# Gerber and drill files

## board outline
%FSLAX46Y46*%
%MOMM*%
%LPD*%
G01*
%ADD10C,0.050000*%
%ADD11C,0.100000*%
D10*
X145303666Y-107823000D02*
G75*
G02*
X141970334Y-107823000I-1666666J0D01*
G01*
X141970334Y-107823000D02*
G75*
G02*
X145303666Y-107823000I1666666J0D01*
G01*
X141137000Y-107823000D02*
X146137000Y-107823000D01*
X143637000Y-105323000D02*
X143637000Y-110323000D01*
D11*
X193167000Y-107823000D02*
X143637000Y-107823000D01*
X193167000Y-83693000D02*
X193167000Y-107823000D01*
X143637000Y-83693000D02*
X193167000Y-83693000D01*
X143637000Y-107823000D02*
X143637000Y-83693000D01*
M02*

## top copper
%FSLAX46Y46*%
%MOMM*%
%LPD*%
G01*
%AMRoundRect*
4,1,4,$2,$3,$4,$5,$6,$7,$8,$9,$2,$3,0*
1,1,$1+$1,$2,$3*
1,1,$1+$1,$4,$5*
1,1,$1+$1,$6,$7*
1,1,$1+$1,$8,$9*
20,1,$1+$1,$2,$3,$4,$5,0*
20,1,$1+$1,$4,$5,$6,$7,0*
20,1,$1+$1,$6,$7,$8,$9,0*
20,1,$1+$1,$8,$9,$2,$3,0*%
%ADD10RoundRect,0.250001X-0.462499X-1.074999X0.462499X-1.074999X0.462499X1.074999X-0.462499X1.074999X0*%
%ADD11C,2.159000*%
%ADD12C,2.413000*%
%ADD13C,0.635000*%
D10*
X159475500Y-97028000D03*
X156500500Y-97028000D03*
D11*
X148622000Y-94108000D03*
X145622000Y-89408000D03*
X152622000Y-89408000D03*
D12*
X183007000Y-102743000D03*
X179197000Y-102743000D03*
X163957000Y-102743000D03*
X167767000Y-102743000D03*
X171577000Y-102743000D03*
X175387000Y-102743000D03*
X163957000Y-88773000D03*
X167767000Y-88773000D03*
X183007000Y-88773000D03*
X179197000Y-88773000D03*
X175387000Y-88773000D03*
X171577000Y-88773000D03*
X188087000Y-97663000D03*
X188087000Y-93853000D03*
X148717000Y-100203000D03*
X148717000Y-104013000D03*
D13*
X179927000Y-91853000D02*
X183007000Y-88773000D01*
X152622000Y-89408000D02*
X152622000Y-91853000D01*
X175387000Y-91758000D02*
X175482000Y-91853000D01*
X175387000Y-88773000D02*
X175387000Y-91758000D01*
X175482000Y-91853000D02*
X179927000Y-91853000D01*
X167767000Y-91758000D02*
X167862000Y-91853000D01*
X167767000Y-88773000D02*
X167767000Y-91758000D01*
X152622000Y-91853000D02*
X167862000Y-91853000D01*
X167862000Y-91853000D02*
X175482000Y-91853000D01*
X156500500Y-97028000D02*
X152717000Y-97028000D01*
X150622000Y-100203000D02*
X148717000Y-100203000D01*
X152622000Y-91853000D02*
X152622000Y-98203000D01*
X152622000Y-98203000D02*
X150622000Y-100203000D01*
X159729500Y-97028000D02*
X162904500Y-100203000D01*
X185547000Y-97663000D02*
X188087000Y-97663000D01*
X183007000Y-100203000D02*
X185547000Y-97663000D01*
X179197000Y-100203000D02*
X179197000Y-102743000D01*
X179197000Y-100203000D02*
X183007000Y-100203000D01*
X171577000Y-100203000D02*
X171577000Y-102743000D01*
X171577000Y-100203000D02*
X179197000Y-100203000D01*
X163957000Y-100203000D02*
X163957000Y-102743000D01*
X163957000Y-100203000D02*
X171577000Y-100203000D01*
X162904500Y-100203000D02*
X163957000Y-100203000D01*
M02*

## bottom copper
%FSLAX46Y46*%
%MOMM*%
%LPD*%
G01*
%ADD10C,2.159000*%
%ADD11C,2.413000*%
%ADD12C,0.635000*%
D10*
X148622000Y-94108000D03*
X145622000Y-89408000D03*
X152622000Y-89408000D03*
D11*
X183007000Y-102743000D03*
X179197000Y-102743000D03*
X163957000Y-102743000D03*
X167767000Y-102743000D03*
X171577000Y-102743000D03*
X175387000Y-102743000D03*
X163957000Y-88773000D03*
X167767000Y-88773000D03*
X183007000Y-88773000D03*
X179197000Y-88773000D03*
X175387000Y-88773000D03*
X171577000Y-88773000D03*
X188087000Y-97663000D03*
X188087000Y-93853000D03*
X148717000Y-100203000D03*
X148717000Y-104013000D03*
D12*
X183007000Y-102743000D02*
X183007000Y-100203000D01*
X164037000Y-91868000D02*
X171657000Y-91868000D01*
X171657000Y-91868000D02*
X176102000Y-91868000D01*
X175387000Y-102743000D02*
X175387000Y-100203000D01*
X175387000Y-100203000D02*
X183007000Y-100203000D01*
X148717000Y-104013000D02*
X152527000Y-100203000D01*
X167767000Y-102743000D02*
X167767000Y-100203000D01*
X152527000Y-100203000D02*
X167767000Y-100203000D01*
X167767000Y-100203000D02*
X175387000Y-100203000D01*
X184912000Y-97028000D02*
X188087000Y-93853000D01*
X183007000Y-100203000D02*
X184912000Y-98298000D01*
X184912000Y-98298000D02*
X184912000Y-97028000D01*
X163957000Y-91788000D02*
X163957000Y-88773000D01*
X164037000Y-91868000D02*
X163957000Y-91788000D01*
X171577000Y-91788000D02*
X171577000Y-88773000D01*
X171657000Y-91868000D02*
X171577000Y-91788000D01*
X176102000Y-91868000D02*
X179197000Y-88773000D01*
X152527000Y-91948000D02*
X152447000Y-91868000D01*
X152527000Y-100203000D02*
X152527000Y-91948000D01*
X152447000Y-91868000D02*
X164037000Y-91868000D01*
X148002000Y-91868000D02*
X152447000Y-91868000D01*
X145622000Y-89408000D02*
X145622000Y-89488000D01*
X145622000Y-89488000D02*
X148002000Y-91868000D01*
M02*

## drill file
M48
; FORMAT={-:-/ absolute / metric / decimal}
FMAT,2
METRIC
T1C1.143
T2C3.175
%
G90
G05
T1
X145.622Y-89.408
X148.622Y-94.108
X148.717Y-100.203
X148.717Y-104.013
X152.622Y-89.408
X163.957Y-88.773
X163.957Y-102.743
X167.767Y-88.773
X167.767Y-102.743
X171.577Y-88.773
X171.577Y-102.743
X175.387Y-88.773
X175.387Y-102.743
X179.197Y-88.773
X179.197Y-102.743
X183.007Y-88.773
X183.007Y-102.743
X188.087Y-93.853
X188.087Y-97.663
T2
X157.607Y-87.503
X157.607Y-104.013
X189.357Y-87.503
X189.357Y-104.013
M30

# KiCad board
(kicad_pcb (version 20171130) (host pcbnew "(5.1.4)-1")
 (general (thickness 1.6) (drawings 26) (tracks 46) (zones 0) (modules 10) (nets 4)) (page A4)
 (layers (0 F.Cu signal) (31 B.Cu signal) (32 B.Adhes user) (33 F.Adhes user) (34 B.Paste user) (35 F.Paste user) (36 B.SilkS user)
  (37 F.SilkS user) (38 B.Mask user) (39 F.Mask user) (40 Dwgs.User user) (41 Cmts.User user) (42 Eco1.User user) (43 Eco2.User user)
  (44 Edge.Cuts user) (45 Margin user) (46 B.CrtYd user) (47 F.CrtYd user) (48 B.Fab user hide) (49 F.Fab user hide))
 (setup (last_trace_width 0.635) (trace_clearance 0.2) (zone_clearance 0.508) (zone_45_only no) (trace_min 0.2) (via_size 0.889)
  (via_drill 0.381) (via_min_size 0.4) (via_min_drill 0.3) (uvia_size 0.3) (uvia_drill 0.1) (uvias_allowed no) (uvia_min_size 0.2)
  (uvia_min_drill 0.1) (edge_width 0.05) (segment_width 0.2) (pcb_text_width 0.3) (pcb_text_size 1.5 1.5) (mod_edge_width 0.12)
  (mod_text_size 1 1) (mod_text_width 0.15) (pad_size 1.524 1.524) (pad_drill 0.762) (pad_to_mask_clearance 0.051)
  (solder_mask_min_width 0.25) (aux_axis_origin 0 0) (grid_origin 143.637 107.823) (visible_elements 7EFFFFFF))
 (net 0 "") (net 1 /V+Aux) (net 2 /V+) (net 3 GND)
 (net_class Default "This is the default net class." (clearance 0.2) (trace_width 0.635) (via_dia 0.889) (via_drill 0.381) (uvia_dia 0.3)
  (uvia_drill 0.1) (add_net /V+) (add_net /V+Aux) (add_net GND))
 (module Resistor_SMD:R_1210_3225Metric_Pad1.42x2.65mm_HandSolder (layer F.Cu) (at 157.988 97.028)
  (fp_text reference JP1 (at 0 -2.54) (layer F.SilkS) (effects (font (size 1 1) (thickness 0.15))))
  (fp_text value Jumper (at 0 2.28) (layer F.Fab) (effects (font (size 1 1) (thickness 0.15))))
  (pad 2 smd roundrect (at 1.4875 0) (size 1.425 2.65) (layers F.Cu F.Paste F.Mask) (roundrect_rratio 0.175439) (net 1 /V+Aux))
  (pad 1 smd roundrect (at -1.4875 0) (size 1.425 2.65) (layers F.Cu F.Paste F.Mask) (roundrect_rratio 0.175439) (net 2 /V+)))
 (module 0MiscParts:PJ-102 (layer F.Cu) (at 137.922 89.408)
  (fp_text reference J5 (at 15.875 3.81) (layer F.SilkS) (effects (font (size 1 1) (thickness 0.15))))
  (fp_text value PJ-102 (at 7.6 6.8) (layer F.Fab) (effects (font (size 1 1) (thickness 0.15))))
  (pad 3 thru_hole circle (at 10.7 4.7) (size 2.159 2.159) (drill 1.143) (layers *.Cu *.Mask))
  (pad 2 thru_hole circle (at 7.7 0) (size 2.159 2.159) (drill 1.143) (layers *.Cu *.Mask) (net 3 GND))
  (pad 1 thru_hole circle (at 14.7 0) (size 2.159 2.159) (drill 1.143) (layers *.Cu *.Mask) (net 2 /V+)))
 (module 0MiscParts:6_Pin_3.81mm (layer F.Cu) (at 173.482 102.743)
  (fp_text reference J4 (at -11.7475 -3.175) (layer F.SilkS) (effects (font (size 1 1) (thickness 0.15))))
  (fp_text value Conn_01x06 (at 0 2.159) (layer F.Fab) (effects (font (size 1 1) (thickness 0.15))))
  (pad 6 thru_hole circle (at 9.525 0) (size 2.413 2.413) (drill 1.143) (layers *.Cu *.Mask) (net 3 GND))
  (pad 5 thru_hole circle (at 5.715 0) (size 2.413 2.413) (drill 1.143) (layers *.Cu *.Mask) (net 1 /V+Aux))
  (pad 1 thru_hole circle (at -9.525 0) (size 2.413 2.413) (drill 1.143) (layers *.Cu *.Mask) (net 1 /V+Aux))
  (pad 2 thru_hole circle (at -5.715 0) (size 2.413 2.413) (drill 1.143) (layers *.Cu *.Mask) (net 3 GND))
  (pad 3 thru_hole circle (at -1.905 0) (size 2.413 2.413) (drill 1.143) (layers *.Cu *.Mask) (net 1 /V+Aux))
  (pad 4 thru_hole circle (at 1.905 0) (size 2.413 2.413) (drill 1.143) (layers *.Cu *.Mask) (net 3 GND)))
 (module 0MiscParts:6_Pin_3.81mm (layer F.Cu) (at 173.482 88.773 180)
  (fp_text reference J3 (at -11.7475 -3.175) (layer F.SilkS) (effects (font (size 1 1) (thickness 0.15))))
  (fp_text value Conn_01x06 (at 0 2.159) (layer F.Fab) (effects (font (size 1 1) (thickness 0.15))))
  (pad 6 thru_hole circle (at 9.525 0 180) (size 2.413 2.413) (drill 1.143) (layers *.Cu *.Mask) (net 3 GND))
  (pad 5 thru_hole circle (at 5.715 0 180) (size 2.413 2.413) (drill 1.143) (layers *.Cu *.Mask) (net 2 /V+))
  (pad 1 thru_hole circle (at -9.525 0 180) (size 2.413 2.413) (drill 1.143) (layers *.Cu *.Mask) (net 2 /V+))
  (pad 2 thru_hole circle (at -5.715 0 180) (size 2.413 2.413) (drill 1.143) (layers *.Cu *.Mask) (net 3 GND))
  (pad 3 thru_hole circle (at -1.905 0 180) (size 2.413 2.413) (drill 1.143) (layers *.Cu *.Mask) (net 2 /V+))
  (pad 4 thru_hole circle (at 1.905 0 180) (size 2.413 2.413) (drill 1.143) (layers *.Cu *.Mask) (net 3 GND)))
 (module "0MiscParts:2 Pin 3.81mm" (layer F.Cu) (at 188.087 95.758 90)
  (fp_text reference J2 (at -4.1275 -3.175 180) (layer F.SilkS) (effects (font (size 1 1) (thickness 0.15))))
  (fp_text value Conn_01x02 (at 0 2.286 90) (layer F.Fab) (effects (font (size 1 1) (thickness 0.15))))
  (pad 1 thru_hole circle (at -1.905 0 90) (size 2.413 2.413) (drill 1.143) (layers *.Cu *.Mask) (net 1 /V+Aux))
  (pad 2 thru_hole circle (at 1.905 0 90) (size 2.413 2.413) (drill 1.143) (layers *.Cu *.Mask) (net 3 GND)))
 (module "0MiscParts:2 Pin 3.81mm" (layer F.Cu) (at 148.717 102.108 270)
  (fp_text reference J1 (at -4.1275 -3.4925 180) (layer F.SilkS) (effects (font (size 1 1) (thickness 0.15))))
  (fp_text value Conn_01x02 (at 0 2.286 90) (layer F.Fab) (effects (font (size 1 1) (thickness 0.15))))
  (pad 1 thru_hole circle (at -1.905 0 270) (size 2.413 2.413) (drill 1.143) (layers *.Cu *.Mask) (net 2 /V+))
  (pad 2 thru_hole circle (at 1.905 0 270) (size 2.413 2.413) (drill 1.143) (layers *.Cu *.Mask) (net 3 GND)))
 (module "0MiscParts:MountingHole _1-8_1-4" (layer F.Cu) (at 189.357 87.503)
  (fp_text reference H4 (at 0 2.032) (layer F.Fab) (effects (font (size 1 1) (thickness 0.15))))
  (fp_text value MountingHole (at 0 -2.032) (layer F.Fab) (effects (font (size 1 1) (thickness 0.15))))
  (pad "" np_thru_hole circle (at 0 0) (size 3.175 3.175) (drill 3.175) (layers *.Cu *.Mask)))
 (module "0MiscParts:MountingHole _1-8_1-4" (layer F.Cu) (at 157.607 87.503)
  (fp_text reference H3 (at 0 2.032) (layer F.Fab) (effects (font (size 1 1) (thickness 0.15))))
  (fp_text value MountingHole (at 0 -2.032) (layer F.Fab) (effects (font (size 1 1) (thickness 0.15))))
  (pad "" np_thru_hole circle (at 0 0) (size 3.175 3.175) (drill 3.175) (layers *.Cu *.Mask)))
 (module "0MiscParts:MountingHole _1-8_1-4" (layer F.Cu) (at 189.357 104.013)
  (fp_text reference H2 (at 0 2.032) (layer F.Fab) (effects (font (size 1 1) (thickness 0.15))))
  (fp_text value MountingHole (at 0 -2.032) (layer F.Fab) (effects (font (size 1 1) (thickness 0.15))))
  (pad "" np_thru_hole circle (at 0 0) (size 3.175 3.175) (drill 3.175) (layers *.Cu *.Mask)))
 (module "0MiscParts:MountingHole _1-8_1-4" (layer F.Cu) (at 157.607 104.013)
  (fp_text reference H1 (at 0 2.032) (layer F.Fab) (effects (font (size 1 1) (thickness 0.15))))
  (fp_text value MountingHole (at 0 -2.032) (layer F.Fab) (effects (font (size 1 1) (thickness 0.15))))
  (pad "" np_thru_hole circle (at 0 0) (size 3.175 3.175) (drill 3.175) (layers *.Cu *.Mask)))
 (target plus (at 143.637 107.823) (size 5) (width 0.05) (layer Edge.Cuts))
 (gr_line (start 193.167 107.823) (end 143.637 107.823) (layer Edge.Cuts) (width 0.1))
 (gr_line (start 193.167 83.693) (end 193.167 107.823) (layer Edge.Cuts) (width 0.1))
 (gr_line (start 143.637 83.693) (end 193.167 83.693) (layer Edge.Cuts) (width 0.1))
 (gr_line (start 143.637 107.823) (end 143.637 83.693) (layer Edge.Cuts) (width 0.1))
 (segment (start 183.007 102.743) (end 183.007 100.203) (width 0.635) (layer B.Cu) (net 3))
 (segment (start 164.037 91.868) (end 171.657 91.868) (width 0.635) (layer B.Cu) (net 3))
 (segment (start 171.657 91.868) (end 176.102 91.868) (width 0.635) (layer B.Cu) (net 3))
 (segment (start 175.387 102.743) (end 175.387 100.203) (width 0.635) (layer B.Cu) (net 3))
 (segment (start 175.387 100.203) (end 183.007 100.203) (width 0.635) (layer B.Cu) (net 3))
 (segment (start 148.717 104.013) (end 152.527 100.203) (width 0.635) (layer B.Cu) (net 3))
 (segment (start 167.767 102.743) (end 167.767 100.203) (width 0.635) (layer B.Cu) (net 3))
 (segment (start 152.527 100.203) (end 167.767 100.203) (width 0.635) (layer B.Cu) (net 3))
 (segment (start 167.767 100.203) (end 175.387 100.203) (width 0.635) (layer B.Cu) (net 3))
 (segment (start 184.912 97.028) (end 188.087 93.853) (width 0.635) (layer B.Cu) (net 3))
 (segment (start 183.007 100.203) (end 184.912 98.298) (width 0.635) (layer B.Cu) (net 3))
 (segment (start 184.912 98.298) (end 184.912 97.028) (width 0.635) (layer B.Cu) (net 3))
 (segment (start 163.957 91.788) (end 163.957 88.773) (width 0.635) (layer B.Cu) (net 3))
 (segment (start 164.037 91.868) (end 163.957 91.788) (width 0.635) (layer B.Cu) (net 3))
 (segment (start 171.577 91.788) (end 171.577 88.773) (width 0.635) (layer B.Cu) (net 3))
 (segment (start 171.657 91.868) (end 171.577 91.788) (width 0.635) (layer B.Cu) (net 3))
 (segment (start 176.102 91.868) (end 179.197 88.773) (width 0.635) (layer B.Cu) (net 3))
 (segment (start 152.527 91.948) (end 152.447 91.868) (width 0.635) (layer B.Cu) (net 3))
 (segment (start 152.527 100.203) (end 152.527 91.948) (width 0.635) (layer B.Cu) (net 3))
 (segment (start 152.447 91.868) (end 164.037 91.868) (width 0.635) (layer B.Cu) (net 3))
 (segment (start 148.002 91.868) (end 152.447 91.868) (width 0.635) (layer B.Cu) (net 3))
 (segment (start 145.622 89.408) (end 145.622 89.488) (width 0.635) (layer B.Cu) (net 3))
 (segment (start 145.622 89.488) (end 148.002 91.868) (width 0.635) (layer B.Cu) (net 3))
 (segment (start 179.927 91.853) (end 183.007 88.773) (width 0.635) (layer F.Cu) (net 2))
 (segment (start 152.622 89.408) (end 152.622 91.853) (width 0.635) (layer F.Cu) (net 2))
 (segment (start 175.387 91.758) (end 175.482 91.853) (width 0.635) (layer F.Cu) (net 2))
 (segment (start 175.387 88.773) (end 175.387 91.758) (width 0.635) (layer F.Cu) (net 2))
 (segment (start 175.482 91.853) (end 179.927 91.853) (width 0.635) (layer F.Cu) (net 2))
 (segment (start 167.767 91.758) (end 167.862 91.853) (width 0.635) (layer F.Cu) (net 2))
 (segment (start 167.767 88.773) (end 167.767 91.758) (width 0.635) (layer F.Cu) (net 2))
 (segment (start 152.622 91.853) (end 167.862 91.853) (width 0.635) (layer F.Cu) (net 2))
 (segment (start 167.862 91.853) (end 175.482 91.853) (width 0.635) (layer F.Cu) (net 2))
 (segment (start 156.5005 97.028) (end 152.717 97.028) (width 0.635) (layer F.Cu) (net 2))
 (segment (start 150.622 100.203) (end 148.717 100.203) (width 0.635) (layer F.Cu) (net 2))
 (segment (start 152.622 91.853) (end 152.622 98.203) (width 0.635) (layer F.Cu) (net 2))
 (segment (start 152.622 98.203) (end 150.622 100.203) (width 0.635) (layer F.Cu) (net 2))
 (segment (start 159.7295 97.028) (end 162.9045 100.203) (width 0.635) (layer F.Cu) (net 1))
 (segment (start 185.547 97.663) (end 188.087 97.663) (width 0.635) (layer F.Cu) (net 1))
 (segment (start 183.007 100.203) (end 185.547 97.663) (width 0.635) (layer F.Cu) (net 1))
 (segment (start 179.197 100.203) (end 179.197 102.743) (width 0.635) (layer F.Cu) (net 1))
 (segment (start 179.197 100.203) (end 183.007 100.203) (width 0.635) (layer F.Cu) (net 1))
 (segment (start 171.577 100.203) (end 171.577 102.743) (width 0.635) (layer F.Cu) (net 1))
 (segment (start 171.577 100.203) (end 179.197 100.203) (width 0.635) (layer F.Cu) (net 1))
 (segment (start 163.957 100.203) (end 163.957 102.743) (width 0.635) (layer F.Cu) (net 1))
 (segment (start 163.957 100.203) (end 171.577 100.203) (width 0.635) (layer F.Cu) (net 1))
 (segment (start 162.9045 100.203) (end 163.957 100.203) (width 0.635) (layer F.Cu) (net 1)))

